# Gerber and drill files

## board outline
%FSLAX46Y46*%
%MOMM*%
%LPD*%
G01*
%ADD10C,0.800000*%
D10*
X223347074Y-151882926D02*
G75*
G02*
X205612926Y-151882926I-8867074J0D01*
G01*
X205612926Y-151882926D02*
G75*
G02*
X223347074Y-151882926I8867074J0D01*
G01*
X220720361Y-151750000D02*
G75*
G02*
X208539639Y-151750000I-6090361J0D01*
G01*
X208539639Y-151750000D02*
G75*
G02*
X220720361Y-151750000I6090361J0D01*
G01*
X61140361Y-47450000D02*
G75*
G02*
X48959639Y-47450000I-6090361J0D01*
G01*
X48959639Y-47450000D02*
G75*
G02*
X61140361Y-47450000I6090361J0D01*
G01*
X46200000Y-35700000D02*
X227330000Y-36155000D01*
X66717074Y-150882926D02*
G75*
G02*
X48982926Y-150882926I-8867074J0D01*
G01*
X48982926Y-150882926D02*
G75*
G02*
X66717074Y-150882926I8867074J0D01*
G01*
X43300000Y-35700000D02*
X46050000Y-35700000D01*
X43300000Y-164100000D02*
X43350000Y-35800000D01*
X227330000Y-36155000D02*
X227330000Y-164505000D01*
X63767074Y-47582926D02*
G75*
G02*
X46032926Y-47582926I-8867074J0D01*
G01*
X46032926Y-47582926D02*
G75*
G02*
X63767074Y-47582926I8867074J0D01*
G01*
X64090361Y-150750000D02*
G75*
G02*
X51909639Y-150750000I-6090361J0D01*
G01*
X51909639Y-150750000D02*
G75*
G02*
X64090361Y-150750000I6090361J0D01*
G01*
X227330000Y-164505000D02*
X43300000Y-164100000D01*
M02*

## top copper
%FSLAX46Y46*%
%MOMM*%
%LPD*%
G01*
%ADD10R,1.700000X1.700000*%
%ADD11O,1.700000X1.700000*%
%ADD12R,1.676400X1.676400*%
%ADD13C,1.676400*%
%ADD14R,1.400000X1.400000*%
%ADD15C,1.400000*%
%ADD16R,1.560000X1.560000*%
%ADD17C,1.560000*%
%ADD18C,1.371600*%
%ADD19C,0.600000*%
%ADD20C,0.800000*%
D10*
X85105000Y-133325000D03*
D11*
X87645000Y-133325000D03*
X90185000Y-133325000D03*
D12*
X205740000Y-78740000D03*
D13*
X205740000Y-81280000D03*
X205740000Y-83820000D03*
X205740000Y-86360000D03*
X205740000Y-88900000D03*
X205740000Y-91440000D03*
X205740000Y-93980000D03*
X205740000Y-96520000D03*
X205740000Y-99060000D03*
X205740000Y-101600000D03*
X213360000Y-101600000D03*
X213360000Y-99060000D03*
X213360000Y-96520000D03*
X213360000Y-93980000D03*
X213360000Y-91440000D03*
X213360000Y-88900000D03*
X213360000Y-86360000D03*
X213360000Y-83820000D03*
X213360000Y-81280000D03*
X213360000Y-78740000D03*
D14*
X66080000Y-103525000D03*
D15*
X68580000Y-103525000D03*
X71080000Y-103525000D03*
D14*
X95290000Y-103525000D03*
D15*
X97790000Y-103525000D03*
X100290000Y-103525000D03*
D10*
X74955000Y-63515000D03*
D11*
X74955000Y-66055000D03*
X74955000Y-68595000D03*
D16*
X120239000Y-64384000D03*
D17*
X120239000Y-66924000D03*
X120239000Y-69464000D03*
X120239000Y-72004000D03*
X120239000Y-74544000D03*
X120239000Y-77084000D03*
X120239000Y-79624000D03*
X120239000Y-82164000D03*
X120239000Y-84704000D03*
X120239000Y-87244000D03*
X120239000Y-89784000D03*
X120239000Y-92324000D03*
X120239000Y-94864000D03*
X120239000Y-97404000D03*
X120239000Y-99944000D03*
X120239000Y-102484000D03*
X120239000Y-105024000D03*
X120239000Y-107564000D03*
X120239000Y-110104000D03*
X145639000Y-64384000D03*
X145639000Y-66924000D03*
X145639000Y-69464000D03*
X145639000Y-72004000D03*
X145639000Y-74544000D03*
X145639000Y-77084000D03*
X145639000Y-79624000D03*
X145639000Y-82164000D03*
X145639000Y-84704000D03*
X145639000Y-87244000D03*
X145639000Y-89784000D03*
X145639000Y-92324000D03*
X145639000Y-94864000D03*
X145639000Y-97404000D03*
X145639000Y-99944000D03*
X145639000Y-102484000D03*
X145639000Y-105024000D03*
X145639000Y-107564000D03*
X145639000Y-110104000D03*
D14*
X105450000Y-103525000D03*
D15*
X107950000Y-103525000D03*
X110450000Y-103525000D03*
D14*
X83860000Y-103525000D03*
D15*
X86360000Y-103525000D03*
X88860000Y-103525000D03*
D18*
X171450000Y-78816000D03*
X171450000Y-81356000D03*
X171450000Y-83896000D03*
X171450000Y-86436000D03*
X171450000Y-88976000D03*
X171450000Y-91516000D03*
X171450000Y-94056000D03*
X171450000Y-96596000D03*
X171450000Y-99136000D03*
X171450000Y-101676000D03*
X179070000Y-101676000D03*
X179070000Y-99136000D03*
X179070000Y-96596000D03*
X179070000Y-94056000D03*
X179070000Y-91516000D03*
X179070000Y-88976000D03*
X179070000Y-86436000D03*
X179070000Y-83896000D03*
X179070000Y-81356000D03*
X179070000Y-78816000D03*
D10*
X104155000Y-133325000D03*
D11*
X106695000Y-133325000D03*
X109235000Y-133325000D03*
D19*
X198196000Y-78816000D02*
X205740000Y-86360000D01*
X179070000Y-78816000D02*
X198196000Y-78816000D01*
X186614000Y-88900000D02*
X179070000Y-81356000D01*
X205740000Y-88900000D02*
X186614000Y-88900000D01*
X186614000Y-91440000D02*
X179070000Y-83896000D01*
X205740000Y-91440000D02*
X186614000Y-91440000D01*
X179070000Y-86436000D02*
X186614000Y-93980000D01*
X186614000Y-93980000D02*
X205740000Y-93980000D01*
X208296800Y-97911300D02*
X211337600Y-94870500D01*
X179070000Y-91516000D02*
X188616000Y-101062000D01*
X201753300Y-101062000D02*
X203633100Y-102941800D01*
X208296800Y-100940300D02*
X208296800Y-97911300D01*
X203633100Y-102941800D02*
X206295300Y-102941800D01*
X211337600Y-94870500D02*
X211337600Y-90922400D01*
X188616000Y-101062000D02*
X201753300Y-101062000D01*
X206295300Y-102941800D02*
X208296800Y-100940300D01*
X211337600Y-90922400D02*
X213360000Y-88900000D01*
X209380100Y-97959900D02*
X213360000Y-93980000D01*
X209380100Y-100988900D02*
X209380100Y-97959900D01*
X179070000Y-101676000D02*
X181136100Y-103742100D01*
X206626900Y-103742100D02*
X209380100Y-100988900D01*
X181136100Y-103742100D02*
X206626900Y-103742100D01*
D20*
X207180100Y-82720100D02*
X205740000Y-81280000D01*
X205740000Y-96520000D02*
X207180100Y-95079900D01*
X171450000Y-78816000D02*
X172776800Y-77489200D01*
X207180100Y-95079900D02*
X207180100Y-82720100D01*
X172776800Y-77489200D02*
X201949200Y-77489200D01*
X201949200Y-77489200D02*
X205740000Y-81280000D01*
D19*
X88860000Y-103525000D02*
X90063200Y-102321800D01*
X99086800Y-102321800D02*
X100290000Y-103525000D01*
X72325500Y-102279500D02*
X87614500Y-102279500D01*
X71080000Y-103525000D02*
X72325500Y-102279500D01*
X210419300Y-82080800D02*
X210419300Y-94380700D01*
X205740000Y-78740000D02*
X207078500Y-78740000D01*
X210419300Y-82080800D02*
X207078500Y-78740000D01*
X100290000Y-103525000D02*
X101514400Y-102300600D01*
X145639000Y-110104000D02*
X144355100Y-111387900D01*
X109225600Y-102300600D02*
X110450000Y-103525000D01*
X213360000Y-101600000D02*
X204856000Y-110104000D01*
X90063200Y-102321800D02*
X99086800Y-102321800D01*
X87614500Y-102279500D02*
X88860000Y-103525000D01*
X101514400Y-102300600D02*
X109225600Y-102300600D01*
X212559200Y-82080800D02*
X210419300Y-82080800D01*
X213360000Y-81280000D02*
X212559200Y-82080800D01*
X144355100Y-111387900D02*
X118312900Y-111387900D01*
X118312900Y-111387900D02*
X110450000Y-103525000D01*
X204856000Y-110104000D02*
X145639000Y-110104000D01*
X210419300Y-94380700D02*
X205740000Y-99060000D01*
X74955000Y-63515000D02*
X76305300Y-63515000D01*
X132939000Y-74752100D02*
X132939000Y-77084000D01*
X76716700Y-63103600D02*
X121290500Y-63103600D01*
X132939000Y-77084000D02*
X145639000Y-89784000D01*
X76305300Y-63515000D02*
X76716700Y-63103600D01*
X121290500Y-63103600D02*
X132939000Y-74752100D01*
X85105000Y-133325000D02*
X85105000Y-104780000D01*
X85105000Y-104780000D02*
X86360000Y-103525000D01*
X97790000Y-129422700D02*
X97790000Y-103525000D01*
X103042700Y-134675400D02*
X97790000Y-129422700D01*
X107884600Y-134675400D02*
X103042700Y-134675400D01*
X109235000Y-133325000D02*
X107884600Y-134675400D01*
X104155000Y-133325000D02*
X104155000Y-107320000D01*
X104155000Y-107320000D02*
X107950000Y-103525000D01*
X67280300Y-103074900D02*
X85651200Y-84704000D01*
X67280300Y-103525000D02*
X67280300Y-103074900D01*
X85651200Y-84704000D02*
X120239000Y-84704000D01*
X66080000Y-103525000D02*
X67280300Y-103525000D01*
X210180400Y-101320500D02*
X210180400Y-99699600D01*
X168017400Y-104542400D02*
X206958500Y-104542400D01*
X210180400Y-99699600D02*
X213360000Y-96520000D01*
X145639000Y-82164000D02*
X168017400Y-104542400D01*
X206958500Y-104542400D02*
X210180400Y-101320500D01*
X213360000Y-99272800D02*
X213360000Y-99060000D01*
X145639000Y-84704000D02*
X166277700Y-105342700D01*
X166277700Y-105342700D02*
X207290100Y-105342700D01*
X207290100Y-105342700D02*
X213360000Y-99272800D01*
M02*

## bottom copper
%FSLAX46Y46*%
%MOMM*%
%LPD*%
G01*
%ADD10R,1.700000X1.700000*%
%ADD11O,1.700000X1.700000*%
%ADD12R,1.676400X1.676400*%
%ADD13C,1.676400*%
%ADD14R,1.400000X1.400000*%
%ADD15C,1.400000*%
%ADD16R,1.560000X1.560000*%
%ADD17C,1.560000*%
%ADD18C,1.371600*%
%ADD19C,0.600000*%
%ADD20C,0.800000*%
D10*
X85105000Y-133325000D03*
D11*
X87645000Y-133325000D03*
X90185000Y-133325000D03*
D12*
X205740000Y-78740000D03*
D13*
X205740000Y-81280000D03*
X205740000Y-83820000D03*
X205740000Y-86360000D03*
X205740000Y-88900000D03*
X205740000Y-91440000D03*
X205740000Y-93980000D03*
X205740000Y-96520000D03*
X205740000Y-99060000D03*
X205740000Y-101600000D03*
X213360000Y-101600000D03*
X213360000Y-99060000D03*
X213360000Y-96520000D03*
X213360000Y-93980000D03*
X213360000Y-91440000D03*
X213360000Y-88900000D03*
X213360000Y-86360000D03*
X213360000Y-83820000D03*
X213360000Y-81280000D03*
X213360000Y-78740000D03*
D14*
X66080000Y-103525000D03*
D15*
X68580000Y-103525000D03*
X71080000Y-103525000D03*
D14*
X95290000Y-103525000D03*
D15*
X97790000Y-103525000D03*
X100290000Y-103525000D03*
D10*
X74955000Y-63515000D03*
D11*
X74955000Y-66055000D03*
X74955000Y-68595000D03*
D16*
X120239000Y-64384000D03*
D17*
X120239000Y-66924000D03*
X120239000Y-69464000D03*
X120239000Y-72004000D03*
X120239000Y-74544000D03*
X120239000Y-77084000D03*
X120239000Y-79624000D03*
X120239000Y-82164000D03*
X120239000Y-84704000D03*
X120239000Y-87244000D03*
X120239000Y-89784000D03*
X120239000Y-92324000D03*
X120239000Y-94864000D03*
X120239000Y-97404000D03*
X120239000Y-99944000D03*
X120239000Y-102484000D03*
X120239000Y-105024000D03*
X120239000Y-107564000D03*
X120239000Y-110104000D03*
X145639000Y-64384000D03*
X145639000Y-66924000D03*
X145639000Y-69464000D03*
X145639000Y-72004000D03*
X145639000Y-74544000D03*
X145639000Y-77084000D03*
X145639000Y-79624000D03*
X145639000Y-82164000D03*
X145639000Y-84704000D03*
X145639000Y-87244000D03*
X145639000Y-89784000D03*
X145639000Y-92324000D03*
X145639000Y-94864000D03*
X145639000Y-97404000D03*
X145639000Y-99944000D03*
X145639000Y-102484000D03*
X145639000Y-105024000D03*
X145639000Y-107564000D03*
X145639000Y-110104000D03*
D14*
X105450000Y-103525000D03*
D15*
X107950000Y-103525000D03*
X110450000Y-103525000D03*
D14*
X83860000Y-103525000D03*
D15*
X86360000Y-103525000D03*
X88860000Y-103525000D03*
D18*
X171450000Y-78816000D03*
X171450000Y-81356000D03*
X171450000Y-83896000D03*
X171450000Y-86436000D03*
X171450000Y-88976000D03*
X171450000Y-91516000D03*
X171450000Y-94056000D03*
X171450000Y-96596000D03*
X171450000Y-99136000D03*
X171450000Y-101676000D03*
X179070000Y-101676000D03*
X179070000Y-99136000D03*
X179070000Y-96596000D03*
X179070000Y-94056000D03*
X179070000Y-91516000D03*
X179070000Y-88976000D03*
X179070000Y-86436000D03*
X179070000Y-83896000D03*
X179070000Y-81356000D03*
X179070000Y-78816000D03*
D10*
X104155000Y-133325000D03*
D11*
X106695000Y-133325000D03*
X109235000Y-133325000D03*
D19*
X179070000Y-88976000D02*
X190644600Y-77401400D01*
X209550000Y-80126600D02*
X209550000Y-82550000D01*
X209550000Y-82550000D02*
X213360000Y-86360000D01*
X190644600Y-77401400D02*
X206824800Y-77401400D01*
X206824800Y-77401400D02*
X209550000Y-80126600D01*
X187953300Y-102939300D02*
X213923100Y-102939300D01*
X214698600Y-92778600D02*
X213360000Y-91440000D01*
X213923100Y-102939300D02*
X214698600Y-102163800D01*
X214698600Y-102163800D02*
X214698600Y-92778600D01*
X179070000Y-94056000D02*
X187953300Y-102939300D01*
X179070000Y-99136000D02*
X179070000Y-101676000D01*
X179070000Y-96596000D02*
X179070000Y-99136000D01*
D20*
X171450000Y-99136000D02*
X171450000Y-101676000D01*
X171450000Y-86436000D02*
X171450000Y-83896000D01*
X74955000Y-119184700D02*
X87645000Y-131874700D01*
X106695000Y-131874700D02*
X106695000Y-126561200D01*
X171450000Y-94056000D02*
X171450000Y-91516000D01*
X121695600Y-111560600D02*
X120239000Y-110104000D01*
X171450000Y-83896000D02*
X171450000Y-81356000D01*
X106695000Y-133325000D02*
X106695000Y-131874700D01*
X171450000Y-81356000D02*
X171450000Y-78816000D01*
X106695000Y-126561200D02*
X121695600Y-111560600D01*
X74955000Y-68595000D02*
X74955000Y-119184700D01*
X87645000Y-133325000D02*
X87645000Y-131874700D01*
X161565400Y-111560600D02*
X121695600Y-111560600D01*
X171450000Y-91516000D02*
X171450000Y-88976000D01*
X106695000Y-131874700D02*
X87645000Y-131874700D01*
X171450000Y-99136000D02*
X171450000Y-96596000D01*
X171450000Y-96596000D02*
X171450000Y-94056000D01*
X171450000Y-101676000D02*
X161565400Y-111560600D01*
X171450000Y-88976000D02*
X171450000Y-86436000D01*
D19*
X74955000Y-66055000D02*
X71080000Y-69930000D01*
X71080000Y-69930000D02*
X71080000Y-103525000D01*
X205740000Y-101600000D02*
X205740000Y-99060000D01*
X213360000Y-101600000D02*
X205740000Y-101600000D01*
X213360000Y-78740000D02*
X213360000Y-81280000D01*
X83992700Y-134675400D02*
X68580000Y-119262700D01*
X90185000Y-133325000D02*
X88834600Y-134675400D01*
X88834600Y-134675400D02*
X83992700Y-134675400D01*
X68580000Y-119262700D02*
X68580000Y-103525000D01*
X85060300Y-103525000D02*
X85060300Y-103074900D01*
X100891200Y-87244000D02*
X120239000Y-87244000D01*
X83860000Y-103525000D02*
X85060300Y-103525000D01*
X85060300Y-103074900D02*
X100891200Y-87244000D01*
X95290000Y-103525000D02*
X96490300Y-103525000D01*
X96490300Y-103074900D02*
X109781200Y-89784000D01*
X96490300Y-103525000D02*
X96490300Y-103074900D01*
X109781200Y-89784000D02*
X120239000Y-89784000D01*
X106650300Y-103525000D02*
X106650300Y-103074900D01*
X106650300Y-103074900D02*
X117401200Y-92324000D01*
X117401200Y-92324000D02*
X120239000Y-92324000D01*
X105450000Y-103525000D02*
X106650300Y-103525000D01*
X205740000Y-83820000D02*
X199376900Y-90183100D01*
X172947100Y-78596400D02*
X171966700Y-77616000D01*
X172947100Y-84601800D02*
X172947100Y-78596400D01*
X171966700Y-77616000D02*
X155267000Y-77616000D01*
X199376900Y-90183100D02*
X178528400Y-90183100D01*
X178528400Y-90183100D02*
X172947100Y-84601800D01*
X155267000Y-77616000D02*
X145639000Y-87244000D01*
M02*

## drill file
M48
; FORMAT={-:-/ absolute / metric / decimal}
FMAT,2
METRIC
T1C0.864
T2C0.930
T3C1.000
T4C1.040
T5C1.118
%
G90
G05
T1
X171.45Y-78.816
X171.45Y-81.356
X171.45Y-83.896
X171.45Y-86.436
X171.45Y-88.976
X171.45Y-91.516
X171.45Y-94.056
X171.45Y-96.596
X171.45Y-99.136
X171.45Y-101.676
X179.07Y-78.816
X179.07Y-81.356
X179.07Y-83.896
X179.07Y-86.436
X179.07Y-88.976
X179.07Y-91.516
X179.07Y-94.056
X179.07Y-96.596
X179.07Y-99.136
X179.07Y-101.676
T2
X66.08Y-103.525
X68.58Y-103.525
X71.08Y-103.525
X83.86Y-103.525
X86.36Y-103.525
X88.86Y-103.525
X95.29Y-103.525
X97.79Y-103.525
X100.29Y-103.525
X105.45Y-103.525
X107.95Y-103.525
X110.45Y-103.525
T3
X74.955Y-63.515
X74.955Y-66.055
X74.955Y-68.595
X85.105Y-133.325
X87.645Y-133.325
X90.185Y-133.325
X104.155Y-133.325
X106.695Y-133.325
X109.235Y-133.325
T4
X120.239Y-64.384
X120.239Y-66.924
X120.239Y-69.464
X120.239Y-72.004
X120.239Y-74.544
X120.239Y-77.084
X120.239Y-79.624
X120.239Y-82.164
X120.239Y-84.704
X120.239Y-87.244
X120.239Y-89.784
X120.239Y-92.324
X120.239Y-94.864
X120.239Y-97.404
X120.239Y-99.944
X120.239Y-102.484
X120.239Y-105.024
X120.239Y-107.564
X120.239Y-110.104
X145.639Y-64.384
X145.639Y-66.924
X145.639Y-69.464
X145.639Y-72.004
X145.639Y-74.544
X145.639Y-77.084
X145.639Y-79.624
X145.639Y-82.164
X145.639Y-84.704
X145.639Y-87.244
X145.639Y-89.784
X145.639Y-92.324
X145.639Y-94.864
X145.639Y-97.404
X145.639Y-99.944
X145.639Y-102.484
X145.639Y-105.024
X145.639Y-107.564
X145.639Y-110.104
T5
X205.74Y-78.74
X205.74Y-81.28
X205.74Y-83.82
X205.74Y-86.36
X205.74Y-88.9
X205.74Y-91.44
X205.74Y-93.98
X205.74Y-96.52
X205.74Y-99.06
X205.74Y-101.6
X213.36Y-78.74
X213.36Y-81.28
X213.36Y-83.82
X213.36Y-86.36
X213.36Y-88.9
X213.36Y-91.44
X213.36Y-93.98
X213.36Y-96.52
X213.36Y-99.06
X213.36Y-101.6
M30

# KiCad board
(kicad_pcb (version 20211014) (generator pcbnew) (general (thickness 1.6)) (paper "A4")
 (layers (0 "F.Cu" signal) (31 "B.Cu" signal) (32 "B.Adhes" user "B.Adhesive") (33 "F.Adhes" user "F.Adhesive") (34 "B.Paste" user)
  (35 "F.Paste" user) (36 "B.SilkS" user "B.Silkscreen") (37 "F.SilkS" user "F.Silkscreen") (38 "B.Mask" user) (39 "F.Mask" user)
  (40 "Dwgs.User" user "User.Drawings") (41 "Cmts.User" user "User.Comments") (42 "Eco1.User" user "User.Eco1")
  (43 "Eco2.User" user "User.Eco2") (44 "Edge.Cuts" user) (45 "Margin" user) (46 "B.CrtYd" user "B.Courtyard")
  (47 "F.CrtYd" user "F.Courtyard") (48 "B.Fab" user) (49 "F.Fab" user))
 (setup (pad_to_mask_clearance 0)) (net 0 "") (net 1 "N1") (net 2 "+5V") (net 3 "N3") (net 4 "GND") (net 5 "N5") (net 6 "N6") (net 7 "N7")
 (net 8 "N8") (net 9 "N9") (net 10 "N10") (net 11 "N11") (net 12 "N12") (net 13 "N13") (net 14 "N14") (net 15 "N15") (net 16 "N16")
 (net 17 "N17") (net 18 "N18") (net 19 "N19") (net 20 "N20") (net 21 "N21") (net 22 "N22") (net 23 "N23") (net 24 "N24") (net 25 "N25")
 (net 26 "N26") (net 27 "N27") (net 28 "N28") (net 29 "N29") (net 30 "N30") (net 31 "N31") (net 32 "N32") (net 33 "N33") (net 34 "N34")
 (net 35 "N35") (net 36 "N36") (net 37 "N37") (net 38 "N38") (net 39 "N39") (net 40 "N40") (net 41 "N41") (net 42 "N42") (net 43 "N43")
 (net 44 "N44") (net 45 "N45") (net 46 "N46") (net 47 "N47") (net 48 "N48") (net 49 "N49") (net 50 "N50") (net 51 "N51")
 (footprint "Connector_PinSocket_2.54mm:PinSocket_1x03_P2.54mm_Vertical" (layer "F.Cu") (at 85.105 133.325 90)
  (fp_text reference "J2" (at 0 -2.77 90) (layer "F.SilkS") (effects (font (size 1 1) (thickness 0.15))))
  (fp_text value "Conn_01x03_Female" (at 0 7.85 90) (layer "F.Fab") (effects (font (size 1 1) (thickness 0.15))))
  (pad "1" thru_hole rect (at 0 0 90) (size 1.7 1.7) (drill 1) (layers *.Cu *.Mask) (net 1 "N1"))
  (pad "2" thru_hole oval (at 0 2.54 90) (size 1.7 1.7) (drill 1) (layers *.Cu *.Mask) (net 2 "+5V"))
  (pad "3" thru_hole oval (at 0 5.08 90) (size 1.7 1.7) (drill 1) (layers *.Cu *.Mask) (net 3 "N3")))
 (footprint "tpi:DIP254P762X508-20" (layer "F.Cu") (at 213.36 101.6)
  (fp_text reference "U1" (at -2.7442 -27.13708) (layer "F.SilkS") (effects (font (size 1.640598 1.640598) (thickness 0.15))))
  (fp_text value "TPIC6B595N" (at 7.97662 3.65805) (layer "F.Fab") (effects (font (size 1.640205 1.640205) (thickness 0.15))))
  (pad "1" thru_hole rect locked (at -7.62 -22.86) (size 1.6764 1.6764) (drill 1.1176) (layers *.Cu *.Mask) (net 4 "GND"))
  (pad "2" thru_hole circle locked (at -7.62 -20.32) (size 1.6764 1.6764) (drill 1.1176) (layers *.Cu *.Mask) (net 2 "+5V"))
  (pad "3" thru_hole circle locked (at -7.62 -17.78) (size 1.6764 1.6764) (drill 1.1176) (layers *.Cu *.Mask) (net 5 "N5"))
  (pad "4" thru_hole circle locked (at -7.62 -15.24) (size 1.6764 1.6764) (drill 1.1176) (layers *.Cu *.Mask) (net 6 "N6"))
  (pad "5" thru_hole circle locked (at -7.62 -12.7) (size 1.6764 1.6764) (drill 1.1176) (layers *.Cu *.Mask) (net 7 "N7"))
  (pad "6" thru_hole circle locked (at -7.62 -10.16) (size 1.6764 1.6764) (drill 1.1176) (layers *.Cu *.Mask) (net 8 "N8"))
  (pad "7" thru_hole circle locked (at -7.62 -7.62) (size 1.6764 1.6764) (drill 1.1176) (layers *.Cu *.Mask) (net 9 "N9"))
  (pad "8" thru_hole circle locked (at -7.62 -5.08) (size 1.6764 1.6764) (drill 1.1176) (layers *.Cu *.Mask) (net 2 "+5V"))
  (pad "9" thru_hole circle locked (at -7.62 -2.54) (size 1.6764 1.6764) (drill 1.1176) (layers *.Cu *.Mask) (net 4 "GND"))
  (pad "10" thru_hole circle locked (at -7.62 0) (size 1.6764 1.6764) (drill 1.1176) (layers *.Cu *.Mask) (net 4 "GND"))
  (pad "11" thru_hole circle locked (at 0 0) (size 1.6764 1.6764) (drill 1.1176) (layers *.Cu *.Mask) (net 4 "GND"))
  (pad "12" thru_hole circle locked (at 0 -2.54) (size 1.6764 1.6764) (drill 1.1176) (layers *.Cu *.Mask) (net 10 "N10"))
  (pad "13" thru_hole circle locked (at 0 -5.08) (size 1.6764 1.6764) (drill 1.1176) (layers *.Cu *.Mask) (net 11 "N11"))
  (pad "14" thru_hole circle locked (at 0 -7.62) (size 1.6764 1.6764) (drill 1.1176) (layers *.Cu *.Mask) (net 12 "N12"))
  (pad "15" thru_hole circle locked (at 0 -10.16) (size 1.6764 1.6764) (drill 1.1176) (layers *.Cu *.Mask) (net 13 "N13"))
  (pad "16" thru_hole circle locked (at 0 -12.7) (size 1.6764 1.6764) (drill 1.1176) (layers *.Cu *.Mask) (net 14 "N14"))
  (pad "17" thru_hole circle locked (at 0 -15.24) (size 1.6764 1.6764) (drill 1.1176) (layers *.Cu *.Mask) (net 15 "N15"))
  (pad "18" thru_hole circle locked (at 0 -17.78) (size 1.6764 1.6764) (drill 1.1176) (layers *.Cu *.Mask) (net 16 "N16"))
  (pad "19" thru_hole circle locked (at 0 -20.32) (size 1.6764 1.6764) (drill 1.1176) (layers *.Cu *.Mask) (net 4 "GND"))
  (pad "20" thru_hole circle locked (at 0 -22.86) (size 1.6764 1.6764) (drill 1.1176) (layers *.Cu *.Mask) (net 4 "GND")))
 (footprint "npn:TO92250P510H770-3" (layer "F.Cu") (at 68.58 102.87)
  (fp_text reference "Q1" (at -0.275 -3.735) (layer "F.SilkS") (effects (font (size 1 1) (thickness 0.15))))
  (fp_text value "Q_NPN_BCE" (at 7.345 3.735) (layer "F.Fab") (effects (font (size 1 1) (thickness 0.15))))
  (pad "1" thru_hole rect locked (at -2.5 0.655) (size 1.4 1.4) (drill 0.93) (layers *.Cu *.Mask) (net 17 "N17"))
  (pad "2" thru_hole circle locked (at 0 0.655) (size 1.4 1.4) (drill 0.93) (layers *.Cu *.Mask) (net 3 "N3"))
  (pad "3" thru_hole circle locked (at 2.5 0.655) (size 1.4 1.4) (drill 0.93) (layers *.Cu *.Mask) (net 4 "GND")))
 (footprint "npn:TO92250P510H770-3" (layer "F.Cu") (at 97.79 102.87)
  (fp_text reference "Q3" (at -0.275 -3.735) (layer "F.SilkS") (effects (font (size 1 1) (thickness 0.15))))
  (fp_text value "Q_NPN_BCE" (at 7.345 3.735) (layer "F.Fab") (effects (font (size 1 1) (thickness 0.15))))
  (pad "1" thru_hole rect locked (at -2.5 0.655) (size 1.4 1.4) (drill 0.93) (layers *.Cu *.Mask) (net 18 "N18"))
  (pad "2" thru_hole circle locked (at 0 0.655) (size 1.4 1.4) (drill 0.93) (layers *.Cu *.Mask) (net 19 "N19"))
  (pad "3" thru_hole circle locked (at 2.5 0.655) (size 1.4 1.4) (drill 0.93) (layers *.Cu *.Mask) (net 4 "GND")))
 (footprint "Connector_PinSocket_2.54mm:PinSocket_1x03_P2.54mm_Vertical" (layer "F.Cu") (at 74.955 63.515)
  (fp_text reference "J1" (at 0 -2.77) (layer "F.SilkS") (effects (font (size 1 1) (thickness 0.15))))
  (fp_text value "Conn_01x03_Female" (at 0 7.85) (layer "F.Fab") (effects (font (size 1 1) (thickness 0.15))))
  (pad "1" thru_hole rect (at 0 0) (size 1.7 1.7) (drill 1) (layers *.Cu *.Mask) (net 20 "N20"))
  (pad "2" thru_hole oval (at 0 2.54) (size 1.7 1.7) (drill 1) (layers *.Cu *.Mask) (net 4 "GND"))
  (pad "3" thru_hole oval (at 0 5.08) (size 1.7 1.7) (drill 1) (layers *.Cu *.Mask) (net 2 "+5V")))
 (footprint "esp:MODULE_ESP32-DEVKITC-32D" (layer "F.Cu") (at 132.939 84.144)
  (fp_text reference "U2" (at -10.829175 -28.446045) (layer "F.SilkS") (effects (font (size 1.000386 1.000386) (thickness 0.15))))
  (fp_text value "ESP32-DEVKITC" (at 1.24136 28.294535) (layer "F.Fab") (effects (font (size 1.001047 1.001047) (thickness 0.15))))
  (pad "1" thru_hole rect locked (at -12.7 -19.76) (size 1.56 1.56) (drill 1.04) (layers *.Cu *.Mask) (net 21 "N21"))
  (pad "2" thru_hole circle locked (at -12.7 -17.22) (size 1.56 1.56) (drill 1.04) (layers *.Cu *.Mask) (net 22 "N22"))
  (pad "3" thru_hole circle locked (at -12.7 -14.68) (size 1.56 1.56) (drill 1.04) (layers *.Cu *.Mask) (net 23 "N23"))
  (pad "4" thru_hole circle locked (at -12.7 -12.14) (size 1.56 1.56) (drill 1.04) (layers *.Cu *.Mask) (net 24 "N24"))
  (pad "5" thru_hole circle locked (at -12.7 -9.6) (size 1.56 1.56) (drill 1.04) (layers *.Cu *.Mask) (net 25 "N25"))
  (pad "6" thru_hole circle locked (at -12.7 -7.06) (size 1.56 1.56) (drill 1.04) (layers *.Cu *.Mask) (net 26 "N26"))
  (pad "7" thru_hole circle locked (at -12.7 -4.52) (size 1.56 1.56) (drill 1.04) (layers *.Cu *.Mask) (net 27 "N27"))
  (pad "8" thru_hole circle locked (at -12.7 -1.98) (size 1.56 1.56) (drill 1.04) (layers *.Cu *.Mask) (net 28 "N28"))
  (pad "9" thru_hole circle locked (at -12.7 0.56) (size 1.56 1.56) (drill 1.04) (layers *.Cu *.Mask) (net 17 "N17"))
  (pad "10" thru_hole circle locked (at -12.7 3.1) (size 1.56 1.56) (drill 1.04) (layers *.Cu *.Mask) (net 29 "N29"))
  (pad "11" thru_hole circle locked (at -12.7 5.64) (size 1.56 1.56) (drill 1.04) (layers *.Cu *.Mask) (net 18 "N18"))
  (pad "12" thru_hole circle locked (at -12.7 8.18) (size 1.56 1.56) (drill 1.04) (layers *.Cu *.Mask) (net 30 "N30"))
  (pad "13" thru_hole circle locked (at -12.7 10.72) (size 1.56 1.56) (drill 1.04) (layers *.Cu *.Mask) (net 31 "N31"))
  (pad "14" thru_hole circle locked (at -12.7 13.26) (size 1.56 1.56) (drill 1.04) (layers *.Cu *.Mask) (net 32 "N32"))
  (pad "15" thru_hole circle locked (at -12.7 15.8) (size 1.56 1.56) (drill 1.04) (layers *.Cu *.Mask) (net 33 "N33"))
  (pad "16" thru_hole circle locked (at -12.7 18.34) (size 1.56 1.56) (drill 1.04) (layers *.Cu *.Mask) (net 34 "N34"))
  (pad "17" thru_hole circle locked (at -12.7 20.88) (size 1.56 1.56) (drill 1.04) (layers *.Cu *.Mask) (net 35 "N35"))
  (pad "18" thru_hole circle locked (at -12.7 23.42) (size 1.56 1.56) (drill 1.04) (layers *.Cu *.Mask) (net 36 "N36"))
  (pad "19" thru_hole circle locked (at -12.7 25.96) (size 1.56 1.56) (drill 1.04) (layers *.Cu *.Mask) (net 2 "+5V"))
  (pad "20" thru_hole circle locked (at 12.7 -19.76) (size 1.56 1.56) (drill 1.04) (layers *.Cu *.Mask) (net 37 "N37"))
  (pad "21" thru_hole circle locked (at 12.7 -17.22) (size 1.56 1.56) (drill 1.04) (layers *.Cu *.Mask) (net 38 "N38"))
  (pad "22" thru_hole circle locked (at 12.7 -14.68) (size 1.56 1.56) (drill 1.04) (layers *.Cu *.Mask) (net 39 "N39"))
  (pad "23" thru_hole circle locked (at 12.7 -12.14) (size 1.56 1.56) (drill 1.04) (layers *.Cu *.Mask) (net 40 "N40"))
  (pad "24" thru_hole circle locked (at 12.7 -9.6) (size 1.56 1.56) (drill 1.04) (layers *.Cu *.Mask) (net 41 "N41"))
  (pad "25" thru_hole circle locked (at 12.7 -7.06) (size 1.56 1.56) (drill 1.04) (layers *.Cu *.Mask) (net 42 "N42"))
  (pad "26" thru_hole circle locked (at 12.7 -4.52) (size 1.56 1.56) (drill 1.04) (layers *.Cu *.Mask) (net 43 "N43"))
  (pad "27" thru_hole circle locked (at 12.7 -1.98) (size 1.56 1.56) (drill 1.04) (layers *.Cu *.Mask) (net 11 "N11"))
  (pad "28" thru_hole circle locked (at 12.7 0.56) (size 1.56 1.56) (drill 1.04) (layers *.Cu *.Mask) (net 10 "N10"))
  (pad "29" thru_hole circle locked (at 12.7 3.1) (size 1.56 1.56) (drill 1.04) (layers *.Cu *.Mask) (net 5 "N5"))
  (pad "30" thru_hole circle locked (at 12.7 5.64) (size 1.56 1.56) (drill 1.04) (layers *.Cu *.Mask) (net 20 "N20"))
  (pad "31" thru_hole circle locked (at 12.7 8.18) (size 1.56 1.56) (drill 1.04) (layers *.Cu *.Mask) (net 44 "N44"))
  (pad "32" thru_hole circle locked (at 12.7 10.72) (size 1.56 1.56) (drill 1.04) (layers *.Cu *.Mask) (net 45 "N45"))
  (pad "33" thru_hole circle locked (at 12.7 13.26) (size 1.56 1.56) (drill 1.04) (layers *.Cu *.Mask) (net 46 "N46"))
  (pad "34" thru_hole circle locked (at 12.7 15.8) (size 1.56 1.56) (drill 1.04) (layers *.Cu *.Mask) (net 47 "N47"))
  (pad "35" thru_hole circle locked (at 12.7 18.34) (size 1.56 1.56) (drill 1.04) (layers *.Cu *.Mask) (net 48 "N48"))
  (pad "36" thru_hole circle locked (at 12.7 20.88) (size 1.56 1.56) (drill 1.04) (layers *.Cu *.Mask) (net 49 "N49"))
  (pad "37" thru_hole circle locked (at 12.7 23.42) (size 1.56 1.56) (drill 1.04) (layers *.Cu *.Mask) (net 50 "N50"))
  (pad "38" thru_hole circle locked (at 12.7 25.96) (size 1.56 1.56) (drill 1.04) (layers *.Cu *.Mask) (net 4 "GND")))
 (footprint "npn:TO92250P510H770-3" (layer "F.Cu") (at 107.95 102.87)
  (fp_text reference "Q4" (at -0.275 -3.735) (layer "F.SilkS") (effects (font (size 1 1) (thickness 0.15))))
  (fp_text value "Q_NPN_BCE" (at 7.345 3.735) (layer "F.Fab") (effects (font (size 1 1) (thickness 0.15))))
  (pad "1" thru_hole rect locked (at -2.5 0.655) (size 1.4 1.4) (drill 0.93) (layers *.Cu *.Mask) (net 30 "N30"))
  (pad "2" thru_hole circle locked (at 0 0.655) (size 1.4 1.4) (drill 0.93) (layers *.Cu *.Mask) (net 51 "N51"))
  (pad "3" thru_hole circle locked (at 2.5 0.655) (size 1.4 1.4) (drill 0.93) (layers *.Cu *.Mask) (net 4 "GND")))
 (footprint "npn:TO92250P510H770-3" (layer "F.Cu") (at 86.36 102.87)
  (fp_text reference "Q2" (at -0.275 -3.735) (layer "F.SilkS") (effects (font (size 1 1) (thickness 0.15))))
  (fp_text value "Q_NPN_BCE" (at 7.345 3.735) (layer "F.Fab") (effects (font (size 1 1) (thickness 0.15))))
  (pad "1" thru_hole rect locked (at -2.5 0.655) (size 1.4 1.4) (drill 0.93) (layers *.Cu *.Mask) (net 29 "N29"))
  (pad "2" thru_hole circle locked (at 0 0.655) (size 1.4 1.4) (drill 0.93) (layers *.Cu *.Mask) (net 1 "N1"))
  (pad "3" thru_hole circle locked (at 2.5 0.655) (size 1.4 1.4) (drill 0.93) (layers *.Cu *.Mask) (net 4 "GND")))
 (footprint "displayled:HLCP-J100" (layer "F.Cu") (at 171.45 78.816)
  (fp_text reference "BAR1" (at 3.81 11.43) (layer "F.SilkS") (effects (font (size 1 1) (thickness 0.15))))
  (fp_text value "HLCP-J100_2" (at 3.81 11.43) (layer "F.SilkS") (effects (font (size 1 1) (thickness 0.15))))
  (pad "1" thru_hole circle locked (at 0 0) (size 1.3716 1.3716) (drill 0.8636) (layers *.Cu *.Mask) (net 2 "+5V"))
  (pad "2" thru_hole circle locked (at 0 2.54) (size 1.3716 1.3716) (drill 0.8636) (layers *.Cu *.Mask) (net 2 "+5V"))
  (pad "3" thru_hole circle locked (at 0 5.08) (size 1.3716 1.3716) (drill 0.8636) (layers *.Cu *.Mask) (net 2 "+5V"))
  (pad "4" thru_hole circle locked (at 0 7.62) (size 1.3716 1.3716) (drill 0.8636) (layers *.Cu *.Mask) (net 2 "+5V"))
  (pad "5" thru_hole circle locked (at 0 10.16) (size 1.3716 1.3716) (drill 0.8636) (layers *.Cu *.Mask) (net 2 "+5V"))
  (pad "6" thru_hole circle locked (at 0 12.7) (size 1.3716 1.3716) (drill 0.8636) (layers *.Cu *.Mask) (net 2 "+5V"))
  (pad "7" thru_hole circle locked (at 0 15.24) (size 1.3716 1.3716) (drill 0.8636) (layers *.Cu *.Mask) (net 2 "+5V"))
  (pad "8" thru_hole circle locked (at 0 17.78) (size 1.3716 1.3716) (drill 0.8636) (layers *.Cu *.Mask) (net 2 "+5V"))
  (pad "9" thru_hole circle locked (at 0 20.32) (size 1.3716 1.3716) (drill 0.8636) (layers *.Cu *.Mask) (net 2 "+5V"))
  (pad "10" thru_hole circle locked (at 0 22.86) (size 1.3716 1.3716) (drill 0.8636) (layers *.Cu *.Mask) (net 2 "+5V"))
  (pad "11" thru_hole circle locked (at 7.62 22.86) (size 1.3716 1.3716) (drill 0.8636) (layers *.Cu *.Mask) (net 12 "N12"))
  (pad "12" thru_hole circle locked (at 7.62 20.32) (size 1.3716 1.3716) (drill 0.8636) (layers *.Cu *.Mask) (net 12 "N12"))
  (pad "13" thru_hole circle locked (at 7.62 17.78) (size 1.3716 1.3716) (drill 0.8636) (layers *.Cu *.Mask) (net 12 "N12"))
  (pad "14" thru_hole circle locked (at 7.62 15.24) (size 1.3716 1.3716) (drill 0.8636) (layers *.Cu *.Mask) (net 13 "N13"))
  (pad "15" thru_hole circle locked (at 7.62 12.7) (size 1.3716 1.3716) (drill 0.8636) (layers *.Cu *.Mask) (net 14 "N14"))
  (pad "16" thru_hole circle locked (at 7.62 10.16) (size 1.3716 1.3716) (drill 0.8636) (layers *.Cu *.Mask) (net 15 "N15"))
  (pad "17" thru_hole circle locked (at 7.62 7.62) (size 1.3716 1.3716) (drill 0.8636) (layers *.Cu *.Mask) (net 9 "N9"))
  (pad "18" thru_hole circle locked (at 7.62 5.08) (size 1.3716 1.3716) (drill 0.8636) (layers *.Cu *.Mask) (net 8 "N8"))
  (pad "19" thru_hole circle locked (at 7.62 2.54) (size 1.3716 1.3716) (drill 0.8636) (layers *.Cu *.Mask) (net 7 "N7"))
  (pad "20" thru_hole circle locked (at 7.62 0) (size 1.3716 1.3716) (drill 0.8636) (layers *.Cu *.Mask) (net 6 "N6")))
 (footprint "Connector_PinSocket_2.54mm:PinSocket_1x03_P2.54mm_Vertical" (layer "F.Cu") (at 104.155 133.325 90)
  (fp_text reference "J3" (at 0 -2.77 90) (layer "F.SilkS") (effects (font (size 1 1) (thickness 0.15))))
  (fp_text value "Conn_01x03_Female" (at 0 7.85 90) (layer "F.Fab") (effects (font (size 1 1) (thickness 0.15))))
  (pad "1" thru_hole rect (at 0 0 90) (size 1.7 1.7) (drill 1) (layers *.Cu *.Mask) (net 51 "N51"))
  (pad "2" thru_hole oval (at 0 2.54 90) (size 1.7 1.7) (drill 1) (layers *.Cu *.Mask) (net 2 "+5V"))
  (pad "3" thru_hole oval (at 0 5.08 90) (size 1.7 1.7) (drill 1) (layers *.Cu *.Mask) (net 19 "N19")))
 (gr_circle (center 214.48 151.882926) (end 223.347074 151.882926) (layer "Edge.Cuts") (width 0.8) (fill none))
 (gr_circle (center 214.63 151.75) (end 220.720361 151.75) (layer "Edge.Cuts") (width 0.8) (fill none))
 (gr_circle (center 55.05 47.45) (end 61.140361 47.45) (layer "Edge.Cuts") (width 0.8) (fill none))
 (gr_line (start 46.2 35.7) (end 227.33 36.155) (layer "Edge.Cuts") (width 0.8))
 (gr_circle (center 57.85 150.882926) (end 66.717074 150.882926) (layer "Edge.Cuts") (width 0.8) (fill none))
 (gr_line (start 43.3 35.7) (end 46.05 35.7) (layer "Edge.Cuts") (width 0.8))
 (gr_line (start 43.3 164.1) (end 43.35 35.8) (layer "Edge.Cuts") (width 0.8))
 (gr_line (start 227.33 36.155) (end 227.33 164.505) (layer "Edge.Cuts") (width 0.8))
 (gr_circle (center 54.9 47.582926) (end 63.767074 47.582926) (layer "Edge.Cuts") (width 0.8) (fill none))
 (gr_circle (center 58 150.75) (end 64.090361 150.75) (layer "Edge.Cuts") (width 0.8) (fill none))
 (gr_line (start 227.33 164.505) (end 43.3 164.1) (layer "Edge.Cuts") (width 0.8))
 (segment (start 198.196 78.816) (end 205.74 86.36) (width 0.6) (layer "F.Cu") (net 6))
 (segment (start 179.07 78.816) (end 198.196 78.816) (width 0.6) (layer "F.Cu") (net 6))
 (segment (start 186.614 88.9) (end 179.07 81.356) (width 0.6) (layer "F.Cu") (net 7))
 (segment (start 205.74 88.9) (end 186.614 88.9) (width 0.6) (layer "F.Cu") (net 7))
 (segment (start 186.614 91.44) (end 179.07 83.896) (width 0.6) (layer "F.Cu") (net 8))
 (segment (start 205.74 91.44) (end 186.614 91.44) (width 0.6) (layer "F.Cu") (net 8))
 (segment (start 179.07 86.436) (end 186.614 93.98) (width 0.6) (layer "F.Cu") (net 9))
 (segment (start 186.614 93.98) (end 205.74 93.98) (width 0.6) (layer "F.Cu") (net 9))
 (segment (start 179.07 88.976) (end 190.6446 77.4014) (width 0.6) (layer "B.Cu") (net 15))
 (segment (start 209.55 80.1266) (end 209.55 82.55) (width 0.6) (layer "B.Cu") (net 15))
 (segment (start 209.55 82.55) (end 213.36 86.36) (width 0.6) (layer "B.Cu") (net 15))
 (segment (start 190.6446 77.4014) (end 206.8248 77.4014) (width 0.6) (layer "B.Cu") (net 15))
 (segment (start 206.8248 77.4014) (end 209.55 80.1266) (width 0.6) (layer "B.Cu") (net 15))
 (segment (start 208.2968 97.9113) (end 211.3376 94.8705) (width 0.6) (layer "F.Cu") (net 14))
 (segment (start 179.07 91.516) (end 188.616 101.062) (width 0.6) (layer "F.Cu") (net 14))
 (segment (start 201.7533 101.062) (end 203.6331 102.9418) (width 0.6) (layer "F.Cu") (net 14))
 (segment (start 208.2968 100.9403) (end 208.2968 97.9113) (width 0.6) (layer "F.Cu") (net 14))
 (segment (start 203.6331 102.9418) (end 206.2953 102.9418) (width 0.6) (layer "F.Cu") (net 14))
 (segment (start 211.3376 94.8705) (end 211.3376 90.9224) (width 0.6) (layer "F.Cu") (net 14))
 (segment (start 188.616 101.062) (end 201.7533 101.062) (width 0.6) (layer "F.Cu") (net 14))
 (segment (start 206.2953 102.9418) (end 208.2968 100.9403) (width 0.6) (layer "F.Cu") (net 14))
 (segment (start 211.3376 90.9224) (end 213.36 88.9) (width 0.6) (layer "F.Cu") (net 14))
 (segment (start 187.9533 102.9393) (end 213.9231 102.9393) (width 0.6) (layer "B.Cu") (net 13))
 (segment (start 214.6986 92.7786) (end 213.36 91.44) (width 0.6) (layer "B.Cu") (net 13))
 (segment (start 213.9231 102.9393) (end 214.6986 102.1638) (width 0.6) (layer "B.Cu") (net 13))
 (segment (start 214.6986 102.1638) (end 214.6986 92.7786) (width 0.6) (layer "B.Cu") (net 13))
 (segment (start 179.07 94.056) (end 187.9533 102.9393) (width 0.6) (layer "B.Cu") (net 13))
 (segment (start 209.3801 97.9599) (end 213.36 93.98) (width 0.6) (layer "F.Cu") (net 12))
 (segment (start 209.3801 100.9889) (end 209.3801 97.9599) (width 0.6) (layer "F.Cu") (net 12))
 (segment (start 179.07 101.676) (end 181.1361 103.7421) (width 0.6) (layer "F.Cu") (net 12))
 (segment (start 206.6269 103.7421) (end 209.3801 100.9889) (width 0.6) (layer "F.Cu") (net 12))
 (segment (start 181.1361 103.7421) (end 206.6269 103.7421) (width 0.6) (layer "F.Cu") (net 12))
 (segment (start 179.07 99.136) (end 179.07 101.676) (width 0.6) (layer "B.Cu") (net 12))
 (segment (start 179.07 96.596) (end 179.07 99.136) (width 0.6) (layer "B.Cu") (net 12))
 (segment (start 207.1801 82.7201) (end 205.74 81.28) (width 0.8) (layer "F.Cu") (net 2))
 (segment (start 205.74 96.52) (end 207.1801 95.0799) (width 0.8) (layer "F.Cu") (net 2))
 (segment (start 171.45 78.816) (end 172.7768 77.4892) (width 0.8) (layer "F.Cu") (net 2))
 (segment (start 207.1801 95.0799) (end 207.1801 82.7201) (width 0.8) (layer "F.Cu") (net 2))
 (segment (start 172.7768 77.4892) (end 201.9492 77.4892) (width 0.8) (layer "F.Cu") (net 2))
 (segment (start 201.9492 77.4892) (end 205.74 81.28) (width 0.8) (layer "F.Cu") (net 2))
 (segment (start 171.45 99.136) (end 171.45 101.676) (width 0.8) (layer "B.Cu") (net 2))
 (segment (start 171.45 86.436) (end 171.45 83.896) (width 0.8) (layer "B.Cu") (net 2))
 (segment (start 74.955 119.1847) (end 87.645 131.8747) (width 0.8) (layer "B.Cu") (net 2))
 (segment (start 106.695 131.8747) (end 106.695 126.5612) (width 0.8) (layer "B.Cu") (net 2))
 (segment (start 171.45 94.056) (end 171.45 91.516) (width 0.8) (layer "B.Cu") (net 2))
 (segment (start 121.6956 111.5606) (end 120.239 110.104) (width 0.8) (layer "B.Cu") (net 2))
 (segment (start 171.45 83.896) (end 171.45 81.356) (width 0.8) (layer "B.Cu") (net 2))
 (segment (start 106.695 133.325) (end 106.695 131.8747) (width 0.8) (layer "B.Cu") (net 2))
 (segment (start 171.45 81.356) (end 171.45 78.816) (width 0.8) (layer "B.Cu") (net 2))
 (segment (start 106.695 126.5612) (end 121.6956 111.5606) (width 0.8) (layer "B.Cu") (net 2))
 (segment (start 74.955 68.595) (end 74.955 119.1847) (width 0.8) (layer "B.Cu") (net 2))
 (segment (start 87.645 133.325) (end 87.645 131.8747) (width 0.8) (layer "B.Cu") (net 2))
 (segment (start 161.5654 111.5606) (end 121.6956 111.5606) (width 0.8) (layer "B.Cu") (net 2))
 (segment (start 171.45 91.516) (end 171.45 88.976) (width 0.8) (layer "B.Cu") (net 2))
 (segment (start 106.695 131.8747) (end 87.645 131.8747) (width 0.8) (layer "B.Cu") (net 2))
 (segment (start 171.45 99.136) (end 171.45 96.596) (width 0.8) (layer "B.Cu") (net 2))
 (segment (start 171.45 96.596) (end 171.45 94.056) (width 0.8) (layer "B.Cu") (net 2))
 (segment (start 171.45 101.676) (end 161.5654 111.5606) (width 0.8) (layer "B.Cu") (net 2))
 (segment (start 171.45 88.976) (end 171.45 86.436) (width 0.8) (layer "B.Cu") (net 2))
 (segment (start 88.86 103.525) (end 90.0632 102.3218) (width 0.6) (layer "F.Cu") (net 4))
 (segment (start 99.0868 102.3218) (end 100.29 103.525) (width 0.6) (layer "F.Cu") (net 4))
 (segment (start 72.3255 102.2795) (end 87.6145 102.2795) (width 0.6) (layer "F.Cu") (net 4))
 (segment (start 71.08 103.525) (end 72.3255 102.2795) (width 0.6) (layer "F.Cu") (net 4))
 (segment (start 210.4193 82.0808) (end 210.4193 94.3807) (width 0.6) (layer "F.Cu") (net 4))
 (segment (start 205.74 78.74) (end 207.0785 78.74) (width 0.6) (layer "F.Cu") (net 4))
 (segment (start 210.4193 82.0808) (end 207.0785 78.74) (width 0.6) (layer "F.Cu") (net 4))
 (segment (start 100.29 103.525) (end 101.5144 102.3006) (width 0.6) (layer "F.Cu") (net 4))
 (segment (start 145.639 110.104) (end 144.3551 111.3879) (width 0.6) (layer "F.Cu") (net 4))
 (segment (start 109.2256 102.3006) (end 110.45 103.525) (width 0.6) (layer "F.Cu") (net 4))
 (segment (start 213.36 101.6) (end 204.856 110.104) (width 0.6) (layer "F.Cu") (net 4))
 (segment (start 90.0632 102.3218) (end 99.0868 102.3218) (width 0.6) (layer "F.Cu") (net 4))
 (segment (start 87.6145 102.2795) (end 88.86 103.525) (width 0.6) (layer "F.Cu") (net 4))
 (segment (start 101.5144 102.3006) (end 109.2256 102.3006) (width 0.6) (layer "F.Cu") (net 4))
 (segment (start 212.5592 82.0808) (end 210.4193 82.0808) (width 0.6) (layer "F.Cu") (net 4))
 (segment (start 213.36 81.28) (end 212.5592 82.0808) (width 0.6) (layer "F.Cu") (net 4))
 (segment (start 144.3551 111.3879) (end 118.3129 111.3879) (width 0.6) (layer "F.Cu") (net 4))
 (segment (start 118.3129 111.3879) (end 110.45 103.525) (width 0.6) (layer "F.Cu") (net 4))
 (segment (start 204.856 110.104) (end 145.639 110.104) (width 0.6) (layer "F.Cu") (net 4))
 (segment (start 210.4193 94.3807) (end 205.74 99.06) (width 0.6) (layer "F.Cu") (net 4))
 (segment (start 74.955 66.055) (end 71.08 69.93) (width 0.6) (layer "B.Cu") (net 4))
 (segment (start 71.08 69.93) (end 71.08 103.525) (width 0.6) (layer "B.Cu") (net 4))
 (segment (start 205.74 101.6) (end 205.74 99.06) (width 0.6) (layer "B.Cu") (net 4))
 (segment (start 213.36 101.6) (end 205.74 101.6) (width 0.6) (layer "B.Cu") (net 4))
 (segment (start 213.36 78.74) (end 213.36 81.28) (width 0.6) (layer "B.Cu") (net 4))
 (segment (start 74.955 63.515) (end 76.3053 63.515) (width 0.6) (layer "F.Cu") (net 20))
 (segment (start 132.939 74.7521) (end 132.939 77.084) (width 0.6) (layer "F.Cu") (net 20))
 (segment (start 76.7167 63.1036) (end 121.2905 63.1036) (width 0.6) (layer "F.Cu") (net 20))
 (segment (start 132.939 77.084) (end 145.639 89.784) (width 0.6) (layer "F.Cu") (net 20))
 (segment (start 76.3053 63.515) (end 76.7167 63.1036) (width 0.6) (layer "F.Cu") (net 20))
 (segment (start 121.2905 63.1036) (end 132.939 74.7521) (width 0.6) (layer "F.Cu") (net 20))
 (segment (start 83.9927 134.6754) (end 68.58 119.2627) (width 0.6) (layer "B.Cu") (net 3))
 (segment (start 90.185 133.325) (end 88.8346 134.6754) (width 0.6) (layer "B.Cu") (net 3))
 (segment (start 88.8346 134.6754) (end 83.9927 134.6754) (width 0.6) (layer "B.Cu") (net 3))
 (segment (start 68.58 119.2627) (end 68.58 103.525) (width 0.6) (layer "B.Cu") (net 3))
 (segment (start 85.105 133.325) (end 85.105 104.78) (width 0.6) (layer "F.Cu") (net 1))
 (segment (start 85.105 104.78) (end 86.36 103.525) (width 0.6) (layer "F.Cu") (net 1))
 (segment (start 97.79 129.4227) (end 97.79 103.525) (width 0.6) (layer "F.Cu") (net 19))
 (segment (start 103.0427 134.6754) (end 97.79 129.4227) (width 0.6) (layer "F.Cu") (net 19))
 (segment (start 107.8846 134.6754) (end 103.0427 134.6754) (width 0.6) (layer "F.Cu") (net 19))
 (segment (start 109.235 133.325) (end 107.8846 134.6754) (width 0.6) (layer "F.Cu") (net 19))
 (segment (start 104.155 133.325) (end 104.155 107.32) (width 0.6) (layer "F.Cu") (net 51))
 (segment (start 104.155 107.32) (end 107.95 103.525) (width 0.6) (layer "F.Cu") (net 51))
 (segment (start 67.2803 103.0749) (end 85.6512 84.704) (width 0.6) (layer "F.Cu") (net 17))
 (segment (start 67.2803 103.525) (end 67.2803 103.0749) (width 0.6) (layer "F.Cu") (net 17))
 (segment (start 85.6512 84.704) (end 120.239 84.704) (width 0.6) (layer "F.Cu") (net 17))
 (segment (start 66.08 103.525) (end 67.2803 103.525) (width 0.6) (layer "F.Cu") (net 17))
 (segment (start 85.0603 103.525) (end 85.0603 103.0749) (width 0.6) (layer "B.Cu") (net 29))
 (segment (start 100.8912 87.244) (end 120.239 87.244) (width 0.6) (layer "B.Cu") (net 29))
 (segment (start 83.86 103.525) (end 85.0603 103.525) (width 0.6) (layer "B.Cu") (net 29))
 (segment (start 85.0603 103.0749) (end 100.8912 87.244) (width 0.6) (layer "B.Cu") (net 29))
 (segment (start 95.29 103.525) (end 96.4903 103.525) (width 0.6) (layer "B.Cu") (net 18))
 (segment (start 96.4903 103.0749) (end 109.7812 89.784) (width 0.6) (layer "B.Cu") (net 18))
 (segment (start 96.4903 103.525) (end 96.4903 103.0749) (width 0.6) (layer "B.Cu") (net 18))
 (segment (start 109.7812 89.784) (end 120.239 89.784) (width 0.6) (layer "B.Cu") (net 18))
 (segment (start 106.6503 103.525) (end 106.6503 103.0749) (width 0.6) (layer "B.Cu") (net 30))
 (segment (start 106.6503 103.0749) (end 117.4012 92.324) (width 0.6) (layer "B.Cu") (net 30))
 (segment (start 117.4012 92.324) (end 120.239 92.324) (width 0.6) (layer "B.Cu") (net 30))
 (segment (start 105.45 103.525) (end 106.6503 103.525) (width 0.6) (layer "B.Cu") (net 30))
 (segment (start 210.1804 101.3205) (end 210.1804 99.6996) (width 0.6) (layer "F.Cu") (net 11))
 (segment (start 168.0174 104.5424) (end 206.9585 104.5424) (width 0.6) (layer "F.Cu") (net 11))
 (segment (start 210.1804 99.6996) (end 213.36 96.52) (width 0.6) (layer "F.Cu") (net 11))
 (segment (start 145.639 82.164) (end 168.0174 104.5424) (width 0.6) (layer "F.Cu") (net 11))
 (segment (start 206.9585 104.5424) (end 210.1804 101.3205) (width 0.6) (layer "F.Cu") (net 11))
 (segment (start 213.36 99.2728) (end 213.36 99.06) (width 0.6) (layer "F.Cu") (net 10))
 (segment (start 145.639 84.704) (end 166.2777 105.3427) (width 0.6) (layer "F.Cu") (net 10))
 (segment (start 166.2777 105.3427) (end 207.2901 105.3427) (width 0.6) (layer "F.Cu") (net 10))
 (segment (start 207.2901 105.3427) (end 213.36 99.2728) (width 0.6) (layer "F.Cu") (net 10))
 (segment (start 205.74 83.82) (end 199.3769 90.1831) (width 0.6) (layer "B.Cu") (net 5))
 (segment (start 172.9471 78.5964) (end 171.9667 77.616) (width 0.6) (layer "B.Cu") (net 5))
 (segment (start 172.9471 84.6018) (end 172.9471 78.5964) (width 0.6) (layer "B.Cu") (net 5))
 (segment (start 171.9667 77.616) (end 155.267 77.616) (width 0.6) (layer "B.Cu") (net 5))
 (segment (start 199.3769 90.1831) (end 178.5284 90.1831) (width 0.6) (layer "B.Cu") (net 5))
 (segment (start 178.5284 90.1831) (end 172.9471 84.6018) (width 0.6) (layer "B.Cu") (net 5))
 (segment (start 155.267 77.616) (end 145.639 87.244) (width 0.6) (layer "B.Cu") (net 5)))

